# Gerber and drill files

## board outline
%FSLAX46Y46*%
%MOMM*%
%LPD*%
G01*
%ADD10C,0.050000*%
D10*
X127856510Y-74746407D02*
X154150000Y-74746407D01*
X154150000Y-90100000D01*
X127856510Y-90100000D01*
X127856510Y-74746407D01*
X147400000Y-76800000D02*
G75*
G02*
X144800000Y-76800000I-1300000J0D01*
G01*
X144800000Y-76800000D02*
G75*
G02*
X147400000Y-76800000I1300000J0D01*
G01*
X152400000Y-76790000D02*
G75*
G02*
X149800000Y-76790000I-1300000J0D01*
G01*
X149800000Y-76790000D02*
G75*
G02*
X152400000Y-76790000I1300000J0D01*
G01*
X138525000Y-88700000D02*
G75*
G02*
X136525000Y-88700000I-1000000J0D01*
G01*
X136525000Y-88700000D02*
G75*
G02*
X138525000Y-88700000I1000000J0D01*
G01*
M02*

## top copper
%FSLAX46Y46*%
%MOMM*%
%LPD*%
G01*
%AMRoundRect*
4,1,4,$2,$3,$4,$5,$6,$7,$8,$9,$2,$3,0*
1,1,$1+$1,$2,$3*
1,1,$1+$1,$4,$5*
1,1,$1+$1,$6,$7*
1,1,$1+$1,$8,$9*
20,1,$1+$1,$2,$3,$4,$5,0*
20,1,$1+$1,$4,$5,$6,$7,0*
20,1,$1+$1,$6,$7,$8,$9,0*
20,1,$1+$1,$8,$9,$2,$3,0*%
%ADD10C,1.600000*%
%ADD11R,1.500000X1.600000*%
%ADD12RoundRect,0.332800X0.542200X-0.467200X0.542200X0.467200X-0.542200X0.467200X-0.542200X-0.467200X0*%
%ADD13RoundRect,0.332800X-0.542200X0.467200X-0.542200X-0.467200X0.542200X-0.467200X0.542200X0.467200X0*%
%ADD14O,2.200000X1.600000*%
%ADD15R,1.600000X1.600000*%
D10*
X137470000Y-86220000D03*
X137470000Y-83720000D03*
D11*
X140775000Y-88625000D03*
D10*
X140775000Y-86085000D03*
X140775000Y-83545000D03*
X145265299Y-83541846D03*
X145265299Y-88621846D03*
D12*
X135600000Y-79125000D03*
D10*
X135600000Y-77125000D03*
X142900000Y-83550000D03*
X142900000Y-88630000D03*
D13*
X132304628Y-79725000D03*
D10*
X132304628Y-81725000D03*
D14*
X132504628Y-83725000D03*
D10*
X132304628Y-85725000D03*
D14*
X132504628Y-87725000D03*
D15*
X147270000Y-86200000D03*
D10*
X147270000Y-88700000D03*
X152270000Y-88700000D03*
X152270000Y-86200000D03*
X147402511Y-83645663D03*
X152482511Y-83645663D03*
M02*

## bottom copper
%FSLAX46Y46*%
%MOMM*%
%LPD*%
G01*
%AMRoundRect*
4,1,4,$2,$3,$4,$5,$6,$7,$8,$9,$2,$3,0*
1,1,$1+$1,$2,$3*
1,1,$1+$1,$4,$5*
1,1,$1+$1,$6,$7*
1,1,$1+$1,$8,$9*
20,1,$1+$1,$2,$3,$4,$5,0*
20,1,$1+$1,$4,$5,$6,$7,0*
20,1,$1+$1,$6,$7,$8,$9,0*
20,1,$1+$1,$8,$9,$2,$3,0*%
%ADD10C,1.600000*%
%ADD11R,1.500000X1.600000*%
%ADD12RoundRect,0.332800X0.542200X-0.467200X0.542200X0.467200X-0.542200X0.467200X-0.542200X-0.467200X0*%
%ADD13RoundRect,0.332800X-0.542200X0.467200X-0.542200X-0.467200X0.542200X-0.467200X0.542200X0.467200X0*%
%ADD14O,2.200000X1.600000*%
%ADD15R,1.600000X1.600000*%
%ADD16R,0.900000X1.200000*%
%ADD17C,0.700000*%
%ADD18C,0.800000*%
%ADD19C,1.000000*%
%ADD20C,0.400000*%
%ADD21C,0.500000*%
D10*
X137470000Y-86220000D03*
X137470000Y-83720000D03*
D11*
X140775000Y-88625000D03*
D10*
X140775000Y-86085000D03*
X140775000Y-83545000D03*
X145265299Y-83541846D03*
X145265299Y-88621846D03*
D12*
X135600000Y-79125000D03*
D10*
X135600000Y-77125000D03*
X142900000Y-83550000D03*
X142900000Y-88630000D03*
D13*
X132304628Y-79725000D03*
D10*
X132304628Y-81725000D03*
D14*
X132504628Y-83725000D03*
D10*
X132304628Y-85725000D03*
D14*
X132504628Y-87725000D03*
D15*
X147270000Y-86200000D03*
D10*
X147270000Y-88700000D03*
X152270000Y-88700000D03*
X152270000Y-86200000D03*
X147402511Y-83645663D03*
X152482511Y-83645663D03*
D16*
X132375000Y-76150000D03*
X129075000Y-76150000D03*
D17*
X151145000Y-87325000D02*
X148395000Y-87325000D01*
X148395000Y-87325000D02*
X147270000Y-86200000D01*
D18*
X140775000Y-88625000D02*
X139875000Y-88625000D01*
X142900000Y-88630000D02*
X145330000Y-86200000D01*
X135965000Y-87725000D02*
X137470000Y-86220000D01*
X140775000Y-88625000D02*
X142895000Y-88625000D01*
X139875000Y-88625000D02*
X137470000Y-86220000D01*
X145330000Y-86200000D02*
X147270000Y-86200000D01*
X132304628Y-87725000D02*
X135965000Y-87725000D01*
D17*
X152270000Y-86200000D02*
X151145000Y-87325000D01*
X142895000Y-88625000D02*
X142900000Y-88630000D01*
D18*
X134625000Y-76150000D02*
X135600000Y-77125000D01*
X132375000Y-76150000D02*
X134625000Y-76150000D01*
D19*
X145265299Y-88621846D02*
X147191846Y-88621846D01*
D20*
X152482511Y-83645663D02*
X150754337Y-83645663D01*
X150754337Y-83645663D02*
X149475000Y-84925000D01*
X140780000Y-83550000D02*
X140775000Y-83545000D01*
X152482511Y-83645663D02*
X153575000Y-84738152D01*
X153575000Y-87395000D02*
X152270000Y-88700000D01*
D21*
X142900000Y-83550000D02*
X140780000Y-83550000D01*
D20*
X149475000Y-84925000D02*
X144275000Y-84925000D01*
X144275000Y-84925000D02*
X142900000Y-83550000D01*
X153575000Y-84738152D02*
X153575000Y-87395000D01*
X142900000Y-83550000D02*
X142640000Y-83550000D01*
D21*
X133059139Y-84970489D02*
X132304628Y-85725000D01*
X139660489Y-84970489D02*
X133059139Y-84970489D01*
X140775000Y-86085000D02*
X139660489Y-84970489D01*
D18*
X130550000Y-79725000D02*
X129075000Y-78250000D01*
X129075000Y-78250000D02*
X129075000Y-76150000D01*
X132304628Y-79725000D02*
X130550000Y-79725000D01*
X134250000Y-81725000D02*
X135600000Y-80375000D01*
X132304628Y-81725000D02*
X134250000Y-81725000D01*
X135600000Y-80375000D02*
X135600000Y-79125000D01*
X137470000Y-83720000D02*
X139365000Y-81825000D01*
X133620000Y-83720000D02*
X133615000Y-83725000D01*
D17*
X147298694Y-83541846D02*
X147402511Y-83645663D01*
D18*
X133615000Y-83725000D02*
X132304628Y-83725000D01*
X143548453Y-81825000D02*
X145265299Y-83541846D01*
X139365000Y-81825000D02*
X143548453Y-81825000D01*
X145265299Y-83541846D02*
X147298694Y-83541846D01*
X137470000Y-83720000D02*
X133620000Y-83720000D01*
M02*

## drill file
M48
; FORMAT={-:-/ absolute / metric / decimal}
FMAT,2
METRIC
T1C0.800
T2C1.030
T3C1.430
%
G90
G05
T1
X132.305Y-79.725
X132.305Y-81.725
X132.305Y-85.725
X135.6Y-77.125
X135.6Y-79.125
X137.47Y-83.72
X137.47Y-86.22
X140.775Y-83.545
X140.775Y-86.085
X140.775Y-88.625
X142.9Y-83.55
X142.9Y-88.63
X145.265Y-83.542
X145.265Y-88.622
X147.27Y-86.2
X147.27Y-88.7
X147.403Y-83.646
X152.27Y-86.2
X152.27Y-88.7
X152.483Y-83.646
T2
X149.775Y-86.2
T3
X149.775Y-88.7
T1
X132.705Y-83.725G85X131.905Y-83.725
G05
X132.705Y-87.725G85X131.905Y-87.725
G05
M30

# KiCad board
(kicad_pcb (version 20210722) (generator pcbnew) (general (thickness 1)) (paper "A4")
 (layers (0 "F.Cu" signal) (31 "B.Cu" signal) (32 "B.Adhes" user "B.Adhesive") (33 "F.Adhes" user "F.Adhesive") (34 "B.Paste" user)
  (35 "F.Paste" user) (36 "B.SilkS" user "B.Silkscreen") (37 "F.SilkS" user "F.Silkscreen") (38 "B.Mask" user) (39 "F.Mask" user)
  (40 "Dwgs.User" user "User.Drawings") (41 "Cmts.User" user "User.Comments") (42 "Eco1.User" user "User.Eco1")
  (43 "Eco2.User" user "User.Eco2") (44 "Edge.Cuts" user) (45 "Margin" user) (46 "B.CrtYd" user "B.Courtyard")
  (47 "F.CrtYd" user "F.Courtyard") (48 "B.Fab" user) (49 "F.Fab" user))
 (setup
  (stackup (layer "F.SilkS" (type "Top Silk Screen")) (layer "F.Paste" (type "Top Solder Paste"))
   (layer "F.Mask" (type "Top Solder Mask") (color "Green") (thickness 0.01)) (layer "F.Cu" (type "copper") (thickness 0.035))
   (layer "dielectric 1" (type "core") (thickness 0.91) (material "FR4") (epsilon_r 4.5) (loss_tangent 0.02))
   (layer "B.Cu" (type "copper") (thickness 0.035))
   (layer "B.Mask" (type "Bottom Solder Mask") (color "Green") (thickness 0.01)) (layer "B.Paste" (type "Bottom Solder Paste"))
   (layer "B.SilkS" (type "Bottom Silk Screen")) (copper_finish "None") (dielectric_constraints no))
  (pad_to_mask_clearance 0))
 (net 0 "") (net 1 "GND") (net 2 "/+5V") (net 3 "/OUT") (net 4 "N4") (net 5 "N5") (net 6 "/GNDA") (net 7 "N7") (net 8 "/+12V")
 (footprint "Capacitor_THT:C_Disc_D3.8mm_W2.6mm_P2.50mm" (layer "F.Cu") (at 137.47 86.22 90)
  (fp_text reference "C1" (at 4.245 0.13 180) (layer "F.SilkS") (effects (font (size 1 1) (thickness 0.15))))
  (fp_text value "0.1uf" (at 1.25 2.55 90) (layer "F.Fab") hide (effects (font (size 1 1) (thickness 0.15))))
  (pad "1" thru_hole circle locked (at 0 0 90) (size 1.6 1.6) (drill 0.8) (layers *.Cu *.Mask) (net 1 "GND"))
  (pad "2" thru_hole circle locked (at 2.5 0 90) (size 1.6 1.6) (drill 0.8) (layers *.Cu *.Mask) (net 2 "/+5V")))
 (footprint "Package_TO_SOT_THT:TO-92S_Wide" (layer "F.Cu") (at 140.775 88.625 90)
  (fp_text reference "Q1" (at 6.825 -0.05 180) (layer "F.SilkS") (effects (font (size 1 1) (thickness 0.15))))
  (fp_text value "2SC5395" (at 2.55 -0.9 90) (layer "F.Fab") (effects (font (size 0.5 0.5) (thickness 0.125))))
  (pad "1" thru_hole rect locked (at 0 0 90) (size 1.6 1.5) (drill 0.8) (layers *.Cu *.Mask) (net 1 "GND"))
  (pad "2" thru_hole circle locked (at 2.54 0 90) (size 1.6 1.6) (drill 0.8) (layers *.Cu *.Mask) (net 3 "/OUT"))
  (pad "3" thru_hole circle locked (at 5.08 0 90) (size 1.6 1.6) (drill 0.8) (layers *.Cu *.Mask) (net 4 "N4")))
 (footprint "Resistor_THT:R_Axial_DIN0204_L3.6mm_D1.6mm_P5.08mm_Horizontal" (layer "F.Cu") (at 145.265299 83.541846 -90)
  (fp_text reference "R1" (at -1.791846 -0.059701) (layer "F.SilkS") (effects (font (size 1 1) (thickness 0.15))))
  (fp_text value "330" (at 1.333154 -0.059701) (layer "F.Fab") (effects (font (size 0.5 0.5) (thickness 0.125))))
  (pad "1" thru_hole circle locked (at 0 0 270) (size 1.6 1.6) (drill 0.8) (layers *.Cu *.Mask) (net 2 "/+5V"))
  (pad "2" thru_hole circle locked (at 5.08 0 270) (size 1.6 1.6) (drill 0.8) (layers *.Cu *.Mask) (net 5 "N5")))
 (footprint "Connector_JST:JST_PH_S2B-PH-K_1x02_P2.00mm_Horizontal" (layer "F.Cu") (at 135.6 79.125 90)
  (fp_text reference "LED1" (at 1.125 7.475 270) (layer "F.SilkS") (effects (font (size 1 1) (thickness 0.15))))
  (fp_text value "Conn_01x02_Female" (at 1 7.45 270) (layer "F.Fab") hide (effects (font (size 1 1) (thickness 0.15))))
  (pad "1" thru_hole roundrect locked (at 0 0 90) (size 1.6 1.75) (drill 0.8) (layers *.Cu *.Mask) (roundrect_rratio 0.208) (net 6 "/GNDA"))
  (pad "2" thru_hole circle locked (at 2 0 90) (size 1.6 1.6) (drill 0.8) (layers *.Cu *.Mask) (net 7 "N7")))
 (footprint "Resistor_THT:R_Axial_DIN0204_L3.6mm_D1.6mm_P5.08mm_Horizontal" (layer "F.Cu") (at 142.9 83.55 -90)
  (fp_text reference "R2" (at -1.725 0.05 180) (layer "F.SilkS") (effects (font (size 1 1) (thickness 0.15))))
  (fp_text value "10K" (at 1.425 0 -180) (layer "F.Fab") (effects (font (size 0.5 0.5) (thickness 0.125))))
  (pad "1" thru_hole circle locked (at 0 0 270) (size 1.6 1.6) (drill 0.8) (layers *.Cu *.Mask) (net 4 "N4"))
  (pad "2" thru_hole circle locked (at 5.08 0 270) (size 1.6 1.6) (drill 0.8) (layers *.Cu *.Mask) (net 1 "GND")))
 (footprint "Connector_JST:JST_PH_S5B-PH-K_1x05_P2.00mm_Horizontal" (layer "F.Cu") (at 132.304628 79.725 -90)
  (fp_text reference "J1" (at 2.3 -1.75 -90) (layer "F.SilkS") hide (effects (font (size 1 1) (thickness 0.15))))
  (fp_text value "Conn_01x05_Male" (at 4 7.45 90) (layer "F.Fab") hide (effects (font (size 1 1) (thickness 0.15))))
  (pad "1" thru_hole roundrect locked (at 0 0 270) (size 1.6 1.75) (drill 0.8) (layers *.Cu *.Mask) (roundrect_rratio 0.208) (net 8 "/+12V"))
  (pad "2" thru_hole circle locked (at 2 0 270) (size 1.6 1.6) (drill 0.8) (layers *.Cu *.Mask) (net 6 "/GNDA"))
  (pad "3" thru_hole oval locked (at 4 0 270) (size 1.6 2.2) (drill oval 0.8 1.6 (offset 0 -0.2)) (layers *.Cu *.Mask) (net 2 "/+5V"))
  (pad "4" thru_hole circle locked (at 6 0 270) (size 1.6 1.6) (drill 0.8) (layers *.Cu *.Mask) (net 3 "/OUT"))
  (pad "5" thru_hole oval locked (at 8 0 270) (size 1.6 2.2) (drill oval 0.8 1.6 (offset 0 -0.2)) (layers *.Cu *.Mask) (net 1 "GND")))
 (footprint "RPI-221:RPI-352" (layer "F.Cu") (at 146.5 89.6)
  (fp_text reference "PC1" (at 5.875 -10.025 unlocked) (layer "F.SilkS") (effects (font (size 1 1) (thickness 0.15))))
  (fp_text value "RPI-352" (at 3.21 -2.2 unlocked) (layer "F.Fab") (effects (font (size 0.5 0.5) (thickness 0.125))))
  (pad "" np_thru_hole circle locked (at 3.275 -3.4) (size 1.03 1.03) (drill 1.03) (layers *.Mask))
  (pad "" np_thru_hole circle locked (at 3.275 -0.9) (size 1.43 1.43) (drill 1.43) (layers *.Mask))
  (pad "1" thru_hole rect locked (at 0.77 -3.4) (size 1.6 1.6) (drill oval 0.8) (layers *.Cu *.Mask) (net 1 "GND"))
  (pad "2" thru_hole circle locked (at 0.77 -0.9) (size 1.6 1.6) (drill oval 0.8) (layers *.Cu *.Mask) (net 5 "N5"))
  (pad "3" thru_hole circle locked (at 5.77 -0.9) (size 1.6 1.6) (drill oval 0.8) (layers *.Cu *.Mask) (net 4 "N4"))
  (pad "4" thru_hole circle locked (at 5.77 -3.4) (size 1.6 1.6) (drill oval 0.8) (layers *.Cu *.Mask) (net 1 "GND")))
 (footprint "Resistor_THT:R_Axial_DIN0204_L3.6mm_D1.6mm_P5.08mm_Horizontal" (layer "F.Cu") (at 147.402511 83.645663)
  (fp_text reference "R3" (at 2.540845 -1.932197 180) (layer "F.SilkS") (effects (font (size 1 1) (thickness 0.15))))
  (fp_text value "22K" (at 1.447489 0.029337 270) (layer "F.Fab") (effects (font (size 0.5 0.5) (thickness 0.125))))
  (pad "1" thru_hole circle locked (at 0 0) (size 1.6 1.6) (drill 0.8) (layers *.Cu *.Mask) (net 2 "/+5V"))
  (pad "2" thru_hole circle locked (at 5.08 0) (size 1.6 1.6) (drill 0.8) (layers *.Cu *.Mask) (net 4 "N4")))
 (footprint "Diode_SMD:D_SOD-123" (layer "B.Cu") (at 130.725 76.15 180)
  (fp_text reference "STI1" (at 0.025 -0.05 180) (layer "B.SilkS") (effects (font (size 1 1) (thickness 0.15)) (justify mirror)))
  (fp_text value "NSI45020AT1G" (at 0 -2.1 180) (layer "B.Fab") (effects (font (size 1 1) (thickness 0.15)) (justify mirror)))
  (pad "1" smd rect locked (at -1.65 0 180) (size 0.9 1.2) (layers "B.Cu" "B.Paste" "B.Mask") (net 7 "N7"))
  (pad "2" smd rect locked (at 1.65 0 180) (size 0.9 1.2) (layers "B.Cu" "B.Paste" "B.Mask") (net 8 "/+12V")))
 (gr_rect (start 127.85651 74.746407) (end 154.15 90.1) (layer "Edge.Cuts") (width 0.05) (fill none))
 (gr_circle (center 146.1 76.8) (end 147.4 76.8) (layer "Edge.Cuts") (width 0.05) (fill none))
 (gr_circle (center 151.1 76.79) (end 152.4 76.79) (layer "Edge.Cuts") (width 0.05) (fill none))
 (gr_circle (center 137.525 88.7) (end 138.525 88.7) (layer "Edge.Cuts") (width 0.05) (fill none))
 (segment (start 151.145 87.325) (end 148.395 87.325) (width 0.7) (layer "B.Cu") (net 1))
 (segment (start 148.395 87.325) (end 147.27 86.2) (width 0.7) (layer "B.Cu") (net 1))
 (segment (start 140.775 88.625) (end 139.875 88.625) (width 0.8) (layer "B.Cu") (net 1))
 (segment (start 142.9 88.63) (end 145.33 86.2) (width 0.8) (layer "B.Cu") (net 1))
 (segment (start 135.965 87.725) (end 137.47 86.22) (width 0.8) (layer "B.Cu") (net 1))
 (segment (start 140.775 88.625) (end 142.895 88.625) (width 0.8) (layer "B.Cu") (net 1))
 (segment (start 139.875 88.625) (end 137.47 86.22) (width 0.8) (layer "B.Cu") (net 1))
 (segment (start 145.33 86.2) (end 147.27 86.2) (width 0.8) (layer "B.Cu") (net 1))
 (segment (start 132.304628 87.725) (end 135.965 87.725) (width 0.8) (layer "B.Cu") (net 1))
 (segment (start 152.27 86.2) (end 151.145 87.325) (width 0.7) (layer "B.Cu") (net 1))
 (segment (start 142.895 88.625) (end 142.9 88.63) (width 0.7) (layer "B.Cu") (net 1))
 (segment (start 134.625 76.15) (end 135.6 77.125) (width 0.8) (layer "B.Cu") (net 7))
 (segment (start 132.375 76.15) (end 134.625 76.15) (width 0.8) (layer "B.Cu") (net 7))
 (segment (start 145.265299 88.621846) (end 147.191846 88.621846) (width 1) (layer "B.Cu") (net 5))
 (segment (start 152.482511 83.645663) (end 150.754337 83.645663) (width 0.4) (layer "B.Cu") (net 4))
 (segment (start 150.754337 83.645663) (end 149.475 84.925) (width 0.4) (layer "B.Cu") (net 4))
 (segment (start 140.78 83.55) (end 140.775 83.545) (width 0.4) (layer "B.Cu") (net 4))
 (segment (start 152.482511 83.645663) (end 153.575 84.738152) (width 0.4) (layer "B.Cu") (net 4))
 (segment (start 153.575 87.395) (end 152.27 88.7) (width 0.4) (layer "B.Cu") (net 4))
 (segment (start 142.9 83.55) (end 140.78 83.55) (width 0.5) (layer "B.Cu") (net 4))
 (segment (start 149.475 84.925) (end 144.275 84.925) (width 0.4) (layer "B.Cu") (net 4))
 (segment (start 144.275 84.925) (end 142.9 83.55) (width 0.4) (layer "B.Cu") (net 4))
 (segment (start 153.575 84.738152) (end 153.575 87.395) (width 0.4) (layer "B.Cu") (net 4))
 (segment (start 142.9 83.55) (end 142.64 83.55) (width 0.4) (layer "B.Cu") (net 4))
 (segment (start 133.059139 84.970489) (end 132.304628 85.725) (width 0.5) (layer "B.Cu") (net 3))
 (segment (start 139.660489 84.970489) (end 133.059139 84.970489) (width 0.5) (layer "B.Cu") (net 3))
 (segment (start 140.775 86.085) (end 139.660489 84.970489) (width 0.5) (layer "B.Cu") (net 3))
 (segment (start 130.55 79.725) (end 129.075 78.25) (width 0.8) (layer "B.Cu") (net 8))
 (segment (start 129.075 78.25) (end 129.075 76.15) (width 0.8) (layer "B.Cu") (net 8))
 (segment (start 132.304628 79.725) (end 130.55 79.725) (width 0.8) (layer "B.Cu") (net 8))
 (segment (start 134.25 81.725) (end 135.6 80.375) (width 0.8) (layer "B.Cu") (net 6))
 (segment (start 132.304628 81.725) (end 134.25 81.725) (width 0.8) (layer "B.Cu") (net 6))
 (segment (start 135.6 80.375) (end 135.6 79.125) (width 0.8) (layer "B.Cu") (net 6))
 (segment (start 137.47 83.72) (end 139.365 81.825) (width 0.8) (layer "B.Cu") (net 2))
 (segment (start 133.62 83.72) (end 133.615 83.725) (width 0.8) (layer "B.Cu") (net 2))
 (segment (start 147.298694 83.541846) (end 147.402511 83.645663) (width 0.7) (layer "B.Cu") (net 2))
 (segment (start 133.615 83.725) (end 132.304628 83.725) (width 0.8) (layer "B.Cu") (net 2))
 (segment (start 143.548453 81.825) (end 145.265299 83.541846) (width 0.8) (layer "B.Cu") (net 2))
 (segment (start 139.365 81.825) (end 143.548453 81.825) (width 0.8) (layer "B.Cu") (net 2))
 (segment (start 145.265299 83.541846) (end 147.298694 83.541846) (width 0.8) (layer "B.Cu") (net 2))
 (segment (start 137.47 83.72) (end 133.62 83.72) (width 0.8) (layer "B.Cu") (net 2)))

